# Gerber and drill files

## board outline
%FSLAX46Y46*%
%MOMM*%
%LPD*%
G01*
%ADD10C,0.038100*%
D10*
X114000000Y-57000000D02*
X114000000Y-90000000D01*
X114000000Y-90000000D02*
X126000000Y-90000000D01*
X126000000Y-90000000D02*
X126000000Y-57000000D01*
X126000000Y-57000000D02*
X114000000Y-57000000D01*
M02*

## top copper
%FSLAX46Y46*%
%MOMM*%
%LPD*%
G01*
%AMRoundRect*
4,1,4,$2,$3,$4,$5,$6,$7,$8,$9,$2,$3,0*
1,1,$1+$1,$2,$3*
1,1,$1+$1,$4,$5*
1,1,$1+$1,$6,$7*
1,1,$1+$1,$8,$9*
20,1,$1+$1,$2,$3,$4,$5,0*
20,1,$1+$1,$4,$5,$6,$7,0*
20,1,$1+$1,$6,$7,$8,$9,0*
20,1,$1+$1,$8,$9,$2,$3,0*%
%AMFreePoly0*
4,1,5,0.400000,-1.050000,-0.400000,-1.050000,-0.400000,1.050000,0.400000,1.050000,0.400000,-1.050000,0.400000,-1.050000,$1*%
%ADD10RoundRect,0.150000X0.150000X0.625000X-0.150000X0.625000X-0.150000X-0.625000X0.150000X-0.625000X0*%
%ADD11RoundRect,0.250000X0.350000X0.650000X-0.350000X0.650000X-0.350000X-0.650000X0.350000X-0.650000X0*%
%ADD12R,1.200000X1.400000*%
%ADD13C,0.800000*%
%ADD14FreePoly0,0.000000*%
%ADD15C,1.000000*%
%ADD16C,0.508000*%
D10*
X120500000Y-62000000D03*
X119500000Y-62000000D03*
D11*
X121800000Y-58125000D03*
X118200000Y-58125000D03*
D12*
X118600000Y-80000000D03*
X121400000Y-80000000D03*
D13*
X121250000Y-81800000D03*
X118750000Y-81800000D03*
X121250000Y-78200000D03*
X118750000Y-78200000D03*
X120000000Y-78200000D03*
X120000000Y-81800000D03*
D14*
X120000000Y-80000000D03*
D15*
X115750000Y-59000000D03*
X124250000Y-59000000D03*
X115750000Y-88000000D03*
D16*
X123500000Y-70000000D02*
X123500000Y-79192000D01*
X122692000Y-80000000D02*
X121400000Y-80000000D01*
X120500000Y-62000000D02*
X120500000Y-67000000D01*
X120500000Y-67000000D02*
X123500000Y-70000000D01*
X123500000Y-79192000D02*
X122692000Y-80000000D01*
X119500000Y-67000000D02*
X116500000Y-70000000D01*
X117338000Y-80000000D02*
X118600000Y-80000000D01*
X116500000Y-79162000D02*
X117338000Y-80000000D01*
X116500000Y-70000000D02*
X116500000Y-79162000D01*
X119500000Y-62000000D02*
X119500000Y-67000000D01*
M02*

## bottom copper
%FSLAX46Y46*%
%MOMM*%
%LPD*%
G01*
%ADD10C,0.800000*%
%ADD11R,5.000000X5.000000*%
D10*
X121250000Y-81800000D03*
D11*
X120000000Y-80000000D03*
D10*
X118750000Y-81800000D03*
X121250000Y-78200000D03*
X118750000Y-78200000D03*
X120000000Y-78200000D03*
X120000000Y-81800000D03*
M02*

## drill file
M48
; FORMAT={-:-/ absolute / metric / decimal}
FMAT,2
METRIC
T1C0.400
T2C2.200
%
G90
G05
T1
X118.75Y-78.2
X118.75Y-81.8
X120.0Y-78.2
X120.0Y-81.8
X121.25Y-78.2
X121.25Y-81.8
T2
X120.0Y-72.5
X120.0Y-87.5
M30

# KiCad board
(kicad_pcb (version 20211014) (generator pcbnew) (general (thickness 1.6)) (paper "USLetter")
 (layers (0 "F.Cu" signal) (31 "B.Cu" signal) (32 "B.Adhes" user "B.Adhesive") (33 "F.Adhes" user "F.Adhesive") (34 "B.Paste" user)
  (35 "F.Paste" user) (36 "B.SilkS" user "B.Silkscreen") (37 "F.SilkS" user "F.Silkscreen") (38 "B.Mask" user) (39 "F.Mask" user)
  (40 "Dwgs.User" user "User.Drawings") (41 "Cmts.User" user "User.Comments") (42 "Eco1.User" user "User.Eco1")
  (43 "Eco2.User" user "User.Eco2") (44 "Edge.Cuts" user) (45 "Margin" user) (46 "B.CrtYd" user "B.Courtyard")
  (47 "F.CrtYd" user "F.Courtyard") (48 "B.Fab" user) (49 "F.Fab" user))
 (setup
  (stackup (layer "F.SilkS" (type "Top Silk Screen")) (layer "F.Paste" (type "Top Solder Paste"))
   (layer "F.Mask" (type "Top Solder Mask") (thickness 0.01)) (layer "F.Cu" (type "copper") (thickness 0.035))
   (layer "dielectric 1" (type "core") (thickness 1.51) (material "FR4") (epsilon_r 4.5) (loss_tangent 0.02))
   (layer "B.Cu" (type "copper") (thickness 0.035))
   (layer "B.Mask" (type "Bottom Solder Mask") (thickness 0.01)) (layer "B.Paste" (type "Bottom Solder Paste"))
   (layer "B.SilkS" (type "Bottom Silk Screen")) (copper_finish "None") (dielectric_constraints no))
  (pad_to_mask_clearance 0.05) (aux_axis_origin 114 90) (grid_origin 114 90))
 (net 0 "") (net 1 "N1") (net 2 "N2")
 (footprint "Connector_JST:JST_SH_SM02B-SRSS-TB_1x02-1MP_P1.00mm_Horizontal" (layer "F.Cu") (at 120 60 180)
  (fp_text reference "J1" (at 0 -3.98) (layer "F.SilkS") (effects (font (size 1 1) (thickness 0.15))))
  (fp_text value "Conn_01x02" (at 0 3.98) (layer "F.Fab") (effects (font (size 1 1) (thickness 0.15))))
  (pad "1" smd roundrect locked (at -0.5 -2 180) (size 0.6 1.55) (layers "F.Cu" "F.Paste" "F.Mask") (roundrect_rratio 0.25) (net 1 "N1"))
  (pad "2" smd roundrect locked (at 0.5 -2 180) (size 0.6 1.55) (layers "F.Cu" "F.Paste" "F.Mask") (roundrect_rratio 0.25) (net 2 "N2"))
  (pad "MP" smd roundrect locked (at -1.8 1.875 180) (size 1.2 1.8) (layers "F.Cu" "F.Paste" "F.Mask") (roundrect_rratio 0.2083333333))
  (pad "MP" smd roundrect locked (at 1.8 1.875 180) (size 1.2 1.8) (layers "F.Cu" "F.Paste" "F.Mask") (roundrect_rratio 0.2083333333)))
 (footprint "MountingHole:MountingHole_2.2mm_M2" (layer "F.Cu") (at 120 87.5)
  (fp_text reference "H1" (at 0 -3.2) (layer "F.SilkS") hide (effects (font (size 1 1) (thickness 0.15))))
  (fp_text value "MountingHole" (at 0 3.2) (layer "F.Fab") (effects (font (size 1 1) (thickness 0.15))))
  (pad "" np_thru_hole circle locked (at 0 0) (size 2.2 2.2) (drill 2.2) (layers *.Cu *.Mask)))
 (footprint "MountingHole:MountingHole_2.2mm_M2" (layer "F.Cu") (at 120 72.5)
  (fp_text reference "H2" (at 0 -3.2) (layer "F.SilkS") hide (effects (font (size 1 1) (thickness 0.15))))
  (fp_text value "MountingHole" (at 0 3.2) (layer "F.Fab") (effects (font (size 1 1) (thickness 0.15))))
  (pad "" np_thru_hole circle locked (at 0 0) (size 2.2 2.2) (drill 2.2) (layers *.Cu *.Mask)))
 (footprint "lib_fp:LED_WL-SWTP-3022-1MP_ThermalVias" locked (layer "F.Cu") (at 120 80)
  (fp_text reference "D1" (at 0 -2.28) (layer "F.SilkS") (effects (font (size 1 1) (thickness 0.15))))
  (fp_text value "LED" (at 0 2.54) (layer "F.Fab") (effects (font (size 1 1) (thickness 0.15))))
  (pad "" smd custom locked (at 0 0) (size 0.7 2) (layers "F.Paste") (zone_connect 0) (options (clearance outline) (anchor rect))
   (primitives))
  (pad "" smd custom locked (at 0 0) (size 0.8 2.1) (layers "F.Mask") (zone_connect 0) (options (clearance outline) (anchor rect))
   (primitives))
  (pad "1" smd rect locked (at -1.4 0) (size 1.2 1.4) (layers "F.Cu" "F.Paste" "F.Mask") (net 2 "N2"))
  (pad "2" smd rect locked (at 1.4 0) (size 1.2 1.4) (layers "F.Cu" "F.Paste" "F.Mask") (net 1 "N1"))
  (pad "MP" thru_hole circle locked (at 1.25 1.8) (size 0.8 0.8) (drill 0.4) (layers *.Cu))
  (pad "MP" smd rect locked (at 0 0) (size 5 5) (layers "B.Cu"))
  (pad "MP" thru_hole circle locked (at -1.25 1.8) (size 0.8 0.8) (drill 0.4) (layers *.Cu))
  (pad "MP" thru_hole circle locked (at 1.25 -1.8) (size 0.8 0.8) (drill 0.4) (layers *.Cu))
  (pad "MP" thru_hole circle locked (at -1.25 -1.8) (size 0.8 0.8) (drill 0.4) (layers *.Cu))
  (pad "MP" thru_hole circle locked (at 0 -1.8) (size 0.8 0.8) (drill 0.4) (layers *.Cu))
  (pad "MP" thru_hole circle locked (at 0 1.8) (size 0.8 0.8) (drill 0.4) (layers *.Cu))
  (pad "MP" smd custom locked (at 0 0) (size 0.8 2.1) (layers "F.Cu") (zone_connect 0) (options (clearance outline) (anchor rect))
   (primitives)))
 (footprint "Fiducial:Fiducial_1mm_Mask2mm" (layer "F.Cu") (at 115.75 59 90)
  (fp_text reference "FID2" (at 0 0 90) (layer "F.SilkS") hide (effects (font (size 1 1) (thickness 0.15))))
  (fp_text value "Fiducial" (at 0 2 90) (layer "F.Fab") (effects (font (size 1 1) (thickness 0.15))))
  (pad "" smd circle locked (at 0 0 90) (size 1 1) (layers "F.Cu" "F.Mask") (solder_mask_margin 0.5) (clearance 0.5)))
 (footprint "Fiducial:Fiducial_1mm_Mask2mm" (layer "F.Cu") (at 124.25 59 90)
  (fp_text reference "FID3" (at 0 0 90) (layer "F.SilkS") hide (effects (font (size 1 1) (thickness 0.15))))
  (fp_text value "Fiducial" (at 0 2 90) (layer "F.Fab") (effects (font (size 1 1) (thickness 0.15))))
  (pad "" smd circle locked (at 0 0 90) (size 1 1) (layers "F.Cu" "F.Mask") (solder_mask_margin 0.5) (clearance 0.5)))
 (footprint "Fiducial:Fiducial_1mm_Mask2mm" (layer "F.Cu") (at 115.75 88 90)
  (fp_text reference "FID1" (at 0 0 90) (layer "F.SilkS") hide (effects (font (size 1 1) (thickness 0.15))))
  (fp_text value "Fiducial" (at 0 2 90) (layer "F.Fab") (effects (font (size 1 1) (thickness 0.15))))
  (pad "" smd circle locked (at 0 0 90) (size 1 1) (layers "F.Cu" "F.Mask") (solder_mask_margin 0.5) (clearance 0.5)))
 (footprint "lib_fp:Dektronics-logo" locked (layer "B.Cu") (at 124.079 80.899 -90)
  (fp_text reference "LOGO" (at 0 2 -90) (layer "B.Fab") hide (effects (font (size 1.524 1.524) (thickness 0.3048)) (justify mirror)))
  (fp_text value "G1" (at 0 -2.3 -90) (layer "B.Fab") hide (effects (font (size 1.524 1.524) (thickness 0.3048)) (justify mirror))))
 (gr_line (start 114 57) (end 114 90) (layer "Edge.Cuts") (width 0.0381))
 (gr_line (start 114 90) (end 126 90) (layer "Edge.Cuts") (width 0.0381))
 (gr_line (start 126 90) (end 126 57) (layer "Edge.Cuts") (width 0.0381))
 (gr_line (start 126 57) (end 114 57) (layer "Edge.Cuts") (width 0.0381))
 (segment (start 123.5 70) (end 123.5 79.192) (width 0.508) (layer "F.Cu") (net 1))
 (segment (start 122.692 80) (end 121.4 80) (width 0.508) (layer "F.Cu") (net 1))
 (segment (start 120.5 62) (end 120.5 67) (width 0.508) (layer "F.Cu") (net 1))
 (segment (start 120.5 67) (end 123.5 70) (width 0.508) (layer "F.Cu") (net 1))
 (segment (start 123.5 79.192) (end 122.692 80) (width 0.508) (layer "F.Cu") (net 1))
 (segment (start 119.5 67) (end 116.5 70) (width 0.508) (layer "F.Cu") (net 2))
 (segment (start 117.338 80) (end 118.6 80) (width 0.508) (layer "F.Cu") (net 2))
 (segment (start 116.5 79.162) (end 117.338 80) (width 0.508) (layer "F.Cu") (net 2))
 (segment (start 116.5 70) (end 116.5 79.162) (width 0.508) (layer "F.Cu") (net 2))
 (segment (start 119.5 62) (end 119.5 67) (width 0.508) (layer "F.Cu") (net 2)))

